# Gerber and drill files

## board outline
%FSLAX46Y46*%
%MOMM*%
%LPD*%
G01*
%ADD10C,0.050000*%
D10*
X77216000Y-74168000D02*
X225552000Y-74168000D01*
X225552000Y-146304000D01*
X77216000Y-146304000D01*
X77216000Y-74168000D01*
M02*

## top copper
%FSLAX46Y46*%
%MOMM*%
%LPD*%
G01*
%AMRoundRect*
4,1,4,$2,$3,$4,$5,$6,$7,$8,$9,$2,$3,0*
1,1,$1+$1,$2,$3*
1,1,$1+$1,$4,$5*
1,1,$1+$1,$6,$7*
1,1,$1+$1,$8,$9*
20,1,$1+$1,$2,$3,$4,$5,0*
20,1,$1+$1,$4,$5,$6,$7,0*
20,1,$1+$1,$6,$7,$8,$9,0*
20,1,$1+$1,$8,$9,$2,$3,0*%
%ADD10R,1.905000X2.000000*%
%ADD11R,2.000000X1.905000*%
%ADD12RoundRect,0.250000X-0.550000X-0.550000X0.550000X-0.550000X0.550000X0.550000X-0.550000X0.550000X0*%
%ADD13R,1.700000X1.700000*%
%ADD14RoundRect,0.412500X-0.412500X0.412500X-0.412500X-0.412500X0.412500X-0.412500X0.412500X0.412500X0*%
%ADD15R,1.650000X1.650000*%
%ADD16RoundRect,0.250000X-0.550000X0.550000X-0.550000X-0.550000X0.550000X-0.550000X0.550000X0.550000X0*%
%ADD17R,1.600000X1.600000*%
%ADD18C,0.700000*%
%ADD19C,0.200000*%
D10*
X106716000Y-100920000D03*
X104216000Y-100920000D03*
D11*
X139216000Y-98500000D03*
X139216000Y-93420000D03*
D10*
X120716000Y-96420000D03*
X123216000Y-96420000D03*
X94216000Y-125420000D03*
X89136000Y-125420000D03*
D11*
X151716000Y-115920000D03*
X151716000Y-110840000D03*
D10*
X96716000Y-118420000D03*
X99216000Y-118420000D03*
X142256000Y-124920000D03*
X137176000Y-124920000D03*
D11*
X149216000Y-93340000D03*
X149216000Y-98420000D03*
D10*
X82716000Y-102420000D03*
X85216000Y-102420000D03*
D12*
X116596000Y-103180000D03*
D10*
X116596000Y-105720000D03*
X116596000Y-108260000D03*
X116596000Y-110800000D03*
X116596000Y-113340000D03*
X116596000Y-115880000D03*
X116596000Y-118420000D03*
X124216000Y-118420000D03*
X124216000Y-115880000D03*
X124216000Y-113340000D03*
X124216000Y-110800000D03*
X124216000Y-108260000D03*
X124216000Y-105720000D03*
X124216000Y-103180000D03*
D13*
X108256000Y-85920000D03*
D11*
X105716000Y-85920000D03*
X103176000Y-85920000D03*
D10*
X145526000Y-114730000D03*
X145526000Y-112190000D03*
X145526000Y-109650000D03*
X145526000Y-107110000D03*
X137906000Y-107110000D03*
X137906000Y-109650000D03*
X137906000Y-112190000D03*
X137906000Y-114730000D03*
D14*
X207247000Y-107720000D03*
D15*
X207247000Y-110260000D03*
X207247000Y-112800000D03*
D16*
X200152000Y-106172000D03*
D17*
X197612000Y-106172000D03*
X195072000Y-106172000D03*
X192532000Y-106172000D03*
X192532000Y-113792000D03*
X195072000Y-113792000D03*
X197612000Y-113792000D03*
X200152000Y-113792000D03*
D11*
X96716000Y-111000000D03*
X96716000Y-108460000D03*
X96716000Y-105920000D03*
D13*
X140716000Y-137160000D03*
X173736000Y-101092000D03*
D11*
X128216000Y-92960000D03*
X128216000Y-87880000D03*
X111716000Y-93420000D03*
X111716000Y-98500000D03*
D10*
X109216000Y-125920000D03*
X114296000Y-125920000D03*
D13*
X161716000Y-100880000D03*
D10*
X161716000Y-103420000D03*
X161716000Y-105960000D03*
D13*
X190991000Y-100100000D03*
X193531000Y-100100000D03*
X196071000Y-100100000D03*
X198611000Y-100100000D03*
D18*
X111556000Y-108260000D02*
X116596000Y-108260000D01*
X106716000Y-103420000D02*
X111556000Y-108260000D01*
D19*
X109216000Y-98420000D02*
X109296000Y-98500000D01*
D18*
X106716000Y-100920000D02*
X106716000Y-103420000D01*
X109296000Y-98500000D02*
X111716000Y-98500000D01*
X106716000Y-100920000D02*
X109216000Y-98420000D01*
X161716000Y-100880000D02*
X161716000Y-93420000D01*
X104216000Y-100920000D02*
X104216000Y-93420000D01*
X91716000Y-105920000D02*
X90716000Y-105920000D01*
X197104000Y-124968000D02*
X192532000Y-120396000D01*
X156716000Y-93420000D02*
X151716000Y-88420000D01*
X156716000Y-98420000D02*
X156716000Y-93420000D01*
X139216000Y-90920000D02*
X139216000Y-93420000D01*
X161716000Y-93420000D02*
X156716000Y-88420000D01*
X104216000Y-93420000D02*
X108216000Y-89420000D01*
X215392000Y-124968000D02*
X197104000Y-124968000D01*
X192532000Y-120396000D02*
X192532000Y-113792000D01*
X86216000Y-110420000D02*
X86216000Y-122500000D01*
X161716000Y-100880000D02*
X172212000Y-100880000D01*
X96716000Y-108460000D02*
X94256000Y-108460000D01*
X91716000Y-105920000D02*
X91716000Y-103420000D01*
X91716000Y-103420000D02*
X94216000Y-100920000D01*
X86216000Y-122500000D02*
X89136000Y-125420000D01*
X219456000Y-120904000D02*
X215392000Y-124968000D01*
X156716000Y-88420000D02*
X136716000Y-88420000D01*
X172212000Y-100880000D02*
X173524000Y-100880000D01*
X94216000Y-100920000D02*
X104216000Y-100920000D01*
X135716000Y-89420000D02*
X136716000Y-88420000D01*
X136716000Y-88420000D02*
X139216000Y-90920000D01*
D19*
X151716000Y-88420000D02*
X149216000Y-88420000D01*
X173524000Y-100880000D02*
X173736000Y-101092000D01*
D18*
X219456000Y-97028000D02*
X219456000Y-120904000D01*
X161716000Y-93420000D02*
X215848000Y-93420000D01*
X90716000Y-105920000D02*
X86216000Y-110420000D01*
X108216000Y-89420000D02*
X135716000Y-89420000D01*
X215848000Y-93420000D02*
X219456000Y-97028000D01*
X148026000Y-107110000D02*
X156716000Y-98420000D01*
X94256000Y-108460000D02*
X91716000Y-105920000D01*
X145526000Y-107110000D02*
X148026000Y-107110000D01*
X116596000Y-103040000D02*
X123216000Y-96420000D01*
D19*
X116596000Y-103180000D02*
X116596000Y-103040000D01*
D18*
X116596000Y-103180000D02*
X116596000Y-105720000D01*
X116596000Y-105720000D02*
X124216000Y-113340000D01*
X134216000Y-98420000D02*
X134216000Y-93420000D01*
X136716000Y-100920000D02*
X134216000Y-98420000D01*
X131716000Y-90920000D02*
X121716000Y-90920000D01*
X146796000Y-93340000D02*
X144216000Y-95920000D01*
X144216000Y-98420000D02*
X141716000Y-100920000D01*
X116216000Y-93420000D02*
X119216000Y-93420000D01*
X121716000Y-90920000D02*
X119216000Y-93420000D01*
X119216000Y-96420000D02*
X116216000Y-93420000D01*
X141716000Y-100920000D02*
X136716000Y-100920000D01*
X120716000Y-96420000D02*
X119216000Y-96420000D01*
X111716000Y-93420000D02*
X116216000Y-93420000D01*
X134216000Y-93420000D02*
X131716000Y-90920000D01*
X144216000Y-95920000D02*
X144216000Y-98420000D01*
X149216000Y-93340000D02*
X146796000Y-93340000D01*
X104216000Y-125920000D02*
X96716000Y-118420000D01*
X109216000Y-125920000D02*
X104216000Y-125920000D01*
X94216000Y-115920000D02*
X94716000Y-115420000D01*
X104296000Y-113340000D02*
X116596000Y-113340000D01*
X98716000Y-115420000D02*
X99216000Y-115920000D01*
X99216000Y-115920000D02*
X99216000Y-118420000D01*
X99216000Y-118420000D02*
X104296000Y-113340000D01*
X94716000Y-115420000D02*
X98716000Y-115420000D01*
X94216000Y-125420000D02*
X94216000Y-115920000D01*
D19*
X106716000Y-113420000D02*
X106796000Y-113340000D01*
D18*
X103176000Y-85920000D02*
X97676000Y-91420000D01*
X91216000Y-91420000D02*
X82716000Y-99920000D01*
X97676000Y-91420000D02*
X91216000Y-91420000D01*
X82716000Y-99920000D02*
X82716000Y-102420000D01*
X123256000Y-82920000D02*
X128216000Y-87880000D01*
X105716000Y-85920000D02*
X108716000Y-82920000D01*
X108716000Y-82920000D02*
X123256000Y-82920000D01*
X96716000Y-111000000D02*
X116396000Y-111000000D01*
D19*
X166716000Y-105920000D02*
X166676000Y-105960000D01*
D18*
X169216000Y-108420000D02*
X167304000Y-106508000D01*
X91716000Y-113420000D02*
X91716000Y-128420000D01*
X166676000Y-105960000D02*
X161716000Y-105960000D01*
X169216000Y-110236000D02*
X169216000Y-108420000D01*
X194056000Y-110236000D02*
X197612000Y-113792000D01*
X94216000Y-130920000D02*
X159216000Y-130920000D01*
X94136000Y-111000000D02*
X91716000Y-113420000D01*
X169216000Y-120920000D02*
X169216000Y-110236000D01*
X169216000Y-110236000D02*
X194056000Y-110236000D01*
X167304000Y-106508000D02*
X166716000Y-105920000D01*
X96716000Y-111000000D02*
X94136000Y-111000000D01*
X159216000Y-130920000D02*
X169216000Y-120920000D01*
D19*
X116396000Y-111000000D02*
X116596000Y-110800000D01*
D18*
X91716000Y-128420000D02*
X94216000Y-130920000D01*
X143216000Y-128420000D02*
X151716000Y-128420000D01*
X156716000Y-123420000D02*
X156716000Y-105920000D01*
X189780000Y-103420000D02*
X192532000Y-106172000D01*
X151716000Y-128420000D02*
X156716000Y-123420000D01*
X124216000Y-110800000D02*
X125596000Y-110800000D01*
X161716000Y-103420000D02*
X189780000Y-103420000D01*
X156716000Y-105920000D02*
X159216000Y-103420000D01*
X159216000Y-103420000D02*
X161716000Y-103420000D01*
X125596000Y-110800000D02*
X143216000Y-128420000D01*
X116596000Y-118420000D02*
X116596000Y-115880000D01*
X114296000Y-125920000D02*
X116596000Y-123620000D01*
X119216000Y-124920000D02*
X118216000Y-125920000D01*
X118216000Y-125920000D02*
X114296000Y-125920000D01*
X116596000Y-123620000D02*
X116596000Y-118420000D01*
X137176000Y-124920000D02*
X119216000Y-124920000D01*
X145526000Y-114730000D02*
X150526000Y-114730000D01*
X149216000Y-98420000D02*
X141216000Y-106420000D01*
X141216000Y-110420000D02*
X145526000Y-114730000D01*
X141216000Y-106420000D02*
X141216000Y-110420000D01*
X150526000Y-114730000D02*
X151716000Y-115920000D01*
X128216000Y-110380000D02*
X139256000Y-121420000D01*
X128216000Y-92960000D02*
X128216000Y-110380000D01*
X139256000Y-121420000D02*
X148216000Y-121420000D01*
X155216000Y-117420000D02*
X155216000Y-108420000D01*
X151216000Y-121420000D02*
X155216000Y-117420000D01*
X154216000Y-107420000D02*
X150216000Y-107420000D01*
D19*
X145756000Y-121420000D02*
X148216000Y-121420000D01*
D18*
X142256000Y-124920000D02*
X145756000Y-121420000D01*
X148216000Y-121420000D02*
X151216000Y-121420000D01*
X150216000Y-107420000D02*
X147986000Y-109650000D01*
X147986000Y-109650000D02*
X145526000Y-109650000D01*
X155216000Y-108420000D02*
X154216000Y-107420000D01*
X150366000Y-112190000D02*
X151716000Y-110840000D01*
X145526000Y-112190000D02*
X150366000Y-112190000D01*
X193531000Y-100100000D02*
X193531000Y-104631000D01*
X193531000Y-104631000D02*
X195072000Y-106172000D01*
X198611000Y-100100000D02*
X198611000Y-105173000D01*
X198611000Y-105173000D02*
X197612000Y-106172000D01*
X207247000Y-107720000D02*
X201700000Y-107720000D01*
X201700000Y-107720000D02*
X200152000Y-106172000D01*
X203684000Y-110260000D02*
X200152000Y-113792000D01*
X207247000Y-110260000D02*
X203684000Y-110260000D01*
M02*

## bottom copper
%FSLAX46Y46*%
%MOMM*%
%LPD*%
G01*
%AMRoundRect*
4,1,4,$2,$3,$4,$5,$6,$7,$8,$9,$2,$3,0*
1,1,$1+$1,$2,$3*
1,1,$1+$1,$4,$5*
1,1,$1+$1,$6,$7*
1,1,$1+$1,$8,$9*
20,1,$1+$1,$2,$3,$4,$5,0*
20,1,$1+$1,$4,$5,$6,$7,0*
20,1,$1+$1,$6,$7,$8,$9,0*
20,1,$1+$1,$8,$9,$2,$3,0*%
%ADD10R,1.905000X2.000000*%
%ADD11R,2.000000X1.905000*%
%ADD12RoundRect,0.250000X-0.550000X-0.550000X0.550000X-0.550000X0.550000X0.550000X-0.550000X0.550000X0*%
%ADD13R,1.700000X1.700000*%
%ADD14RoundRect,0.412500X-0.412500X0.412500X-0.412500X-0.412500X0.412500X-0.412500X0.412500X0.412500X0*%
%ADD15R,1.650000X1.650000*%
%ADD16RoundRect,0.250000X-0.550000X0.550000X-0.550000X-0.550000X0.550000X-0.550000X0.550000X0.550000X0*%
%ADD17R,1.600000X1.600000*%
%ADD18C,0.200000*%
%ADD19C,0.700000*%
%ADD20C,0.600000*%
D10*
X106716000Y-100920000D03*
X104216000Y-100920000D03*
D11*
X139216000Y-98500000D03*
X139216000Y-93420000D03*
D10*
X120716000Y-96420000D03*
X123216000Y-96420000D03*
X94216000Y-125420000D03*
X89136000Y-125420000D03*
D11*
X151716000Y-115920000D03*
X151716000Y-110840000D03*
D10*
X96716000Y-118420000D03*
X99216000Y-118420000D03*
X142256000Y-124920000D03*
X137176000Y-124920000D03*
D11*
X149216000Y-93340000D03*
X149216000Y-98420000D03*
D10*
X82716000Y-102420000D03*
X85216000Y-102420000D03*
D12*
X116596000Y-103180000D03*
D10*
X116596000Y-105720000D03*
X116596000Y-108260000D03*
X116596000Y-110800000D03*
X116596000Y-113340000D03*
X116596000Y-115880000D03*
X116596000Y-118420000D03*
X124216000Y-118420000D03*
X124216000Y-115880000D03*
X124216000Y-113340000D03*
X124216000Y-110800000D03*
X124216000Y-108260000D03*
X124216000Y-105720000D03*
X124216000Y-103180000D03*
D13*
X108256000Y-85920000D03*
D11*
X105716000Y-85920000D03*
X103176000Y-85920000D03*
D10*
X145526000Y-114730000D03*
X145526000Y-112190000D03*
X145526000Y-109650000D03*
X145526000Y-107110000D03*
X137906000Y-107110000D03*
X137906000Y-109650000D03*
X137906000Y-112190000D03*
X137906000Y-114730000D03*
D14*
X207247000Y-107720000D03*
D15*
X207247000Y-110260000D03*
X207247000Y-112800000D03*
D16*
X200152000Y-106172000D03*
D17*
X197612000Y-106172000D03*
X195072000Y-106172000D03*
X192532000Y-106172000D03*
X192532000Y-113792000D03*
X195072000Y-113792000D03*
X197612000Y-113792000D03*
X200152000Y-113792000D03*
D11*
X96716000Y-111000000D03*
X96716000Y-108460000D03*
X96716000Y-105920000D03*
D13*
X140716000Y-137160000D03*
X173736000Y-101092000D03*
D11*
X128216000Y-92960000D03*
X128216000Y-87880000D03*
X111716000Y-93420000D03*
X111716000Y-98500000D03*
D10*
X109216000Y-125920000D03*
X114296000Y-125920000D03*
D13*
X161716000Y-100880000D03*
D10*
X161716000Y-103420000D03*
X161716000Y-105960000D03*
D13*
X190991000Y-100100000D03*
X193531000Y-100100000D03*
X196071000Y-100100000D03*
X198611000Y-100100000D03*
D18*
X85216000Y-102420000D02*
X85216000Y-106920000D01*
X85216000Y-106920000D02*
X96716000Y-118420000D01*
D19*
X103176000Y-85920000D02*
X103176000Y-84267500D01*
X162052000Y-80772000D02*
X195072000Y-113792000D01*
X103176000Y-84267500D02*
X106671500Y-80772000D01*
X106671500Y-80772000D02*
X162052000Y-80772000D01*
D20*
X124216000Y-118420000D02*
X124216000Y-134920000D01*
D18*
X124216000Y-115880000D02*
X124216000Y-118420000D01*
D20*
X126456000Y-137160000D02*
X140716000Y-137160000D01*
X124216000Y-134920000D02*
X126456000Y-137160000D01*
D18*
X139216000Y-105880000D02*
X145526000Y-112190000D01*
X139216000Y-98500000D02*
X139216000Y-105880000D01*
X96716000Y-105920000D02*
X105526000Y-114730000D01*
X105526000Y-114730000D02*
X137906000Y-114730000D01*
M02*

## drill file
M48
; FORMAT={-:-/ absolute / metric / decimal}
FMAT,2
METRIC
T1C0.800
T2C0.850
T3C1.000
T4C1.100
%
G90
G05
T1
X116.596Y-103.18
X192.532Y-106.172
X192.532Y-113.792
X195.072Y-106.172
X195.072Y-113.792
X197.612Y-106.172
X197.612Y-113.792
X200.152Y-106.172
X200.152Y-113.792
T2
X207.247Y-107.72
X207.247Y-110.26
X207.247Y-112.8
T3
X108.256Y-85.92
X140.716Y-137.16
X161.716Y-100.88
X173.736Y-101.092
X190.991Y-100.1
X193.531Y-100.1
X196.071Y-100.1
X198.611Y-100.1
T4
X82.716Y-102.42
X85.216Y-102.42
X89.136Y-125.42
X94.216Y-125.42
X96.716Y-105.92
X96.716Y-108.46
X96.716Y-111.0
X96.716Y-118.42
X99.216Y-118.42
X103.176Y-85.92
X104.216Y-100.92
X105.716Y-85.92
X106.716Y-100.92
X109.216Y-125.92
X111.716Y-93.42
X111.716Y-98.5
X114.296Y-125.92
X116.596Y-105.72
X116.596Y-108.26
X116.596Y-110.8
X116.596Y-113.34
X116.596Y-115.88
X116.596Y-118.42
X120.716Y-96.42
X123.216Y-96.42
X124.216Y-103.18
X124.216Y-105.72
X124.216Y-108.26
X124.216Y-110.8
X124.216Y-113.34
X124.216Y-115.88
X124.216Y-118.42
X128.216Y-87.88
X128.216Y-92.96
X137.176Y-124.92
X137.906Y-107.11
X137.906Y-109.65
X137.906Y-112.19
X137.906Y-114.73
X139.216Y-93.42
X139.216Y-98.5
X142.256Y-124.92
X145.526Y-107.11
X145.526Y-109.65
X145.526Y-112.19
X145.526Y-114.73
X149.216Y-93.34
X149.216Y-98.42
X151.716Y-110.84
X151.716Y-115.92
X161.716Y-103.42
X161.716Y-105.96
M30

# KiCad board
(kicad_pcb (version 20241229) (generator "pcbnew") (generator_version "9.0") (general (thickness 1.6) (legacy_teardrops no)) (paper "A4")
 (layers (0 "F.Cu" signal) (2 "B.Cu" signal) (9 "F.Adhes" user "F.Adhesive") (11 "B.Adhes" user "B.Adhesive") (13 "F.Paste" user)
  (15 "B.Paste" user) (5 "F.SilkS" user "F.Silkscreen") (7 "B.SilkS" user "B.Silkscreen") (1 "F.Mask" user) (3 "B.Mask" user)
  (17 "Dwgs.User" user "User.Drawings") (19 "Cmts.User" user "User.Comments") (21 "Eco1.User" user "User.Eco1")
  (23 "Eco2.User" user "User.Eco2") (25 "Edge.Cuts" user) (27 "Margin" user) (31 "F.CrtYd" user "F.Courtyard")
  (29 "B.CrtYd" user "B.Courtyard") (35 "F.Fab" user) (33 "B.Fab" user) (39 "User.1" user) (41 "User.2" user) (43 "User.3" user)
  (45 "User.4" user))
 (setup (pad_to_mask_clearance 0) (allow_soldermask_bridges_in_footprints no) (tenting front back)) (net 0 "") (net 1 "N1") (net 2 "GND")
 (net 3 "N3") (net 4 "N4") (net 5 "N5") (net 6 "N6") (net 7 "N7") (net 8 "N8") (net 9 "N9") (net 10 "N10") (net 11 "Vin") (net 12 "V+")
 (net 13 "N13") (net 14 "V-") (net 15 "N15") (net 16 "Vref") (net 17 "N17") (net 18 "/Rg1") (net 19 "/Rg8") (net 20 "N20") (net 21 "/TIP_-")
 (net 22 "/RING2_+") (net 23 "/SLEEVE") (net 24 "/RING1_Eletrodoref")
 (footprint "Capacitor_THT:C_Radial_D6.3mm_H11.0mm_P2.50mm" (layer "F.Cu") (at 106.716 100.92 180)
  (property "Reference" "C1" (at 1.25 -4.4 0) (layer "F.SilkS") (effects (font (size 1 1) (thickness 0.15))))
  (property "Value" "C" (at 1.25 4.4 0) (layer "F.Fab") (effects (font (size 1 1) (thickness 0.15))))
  (pad "1" thru_hole rect (at 0 0 180) (size 1.905 2) (drill 1.1) (layers "*.Cu" "*.Mask") (remove_unused_layers no) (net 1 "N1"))
  (pad "2" thru_hole rect (at 2.5 0 180) (size 1.905 2) (drill 1.1) (layers "*.Cu" "*.Mask") (remove_unused_layers no) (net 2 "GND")))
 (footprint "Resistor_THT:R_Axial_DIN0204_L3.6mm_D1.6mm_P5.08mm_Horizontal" (layer "F.Cu") (at 139.216 98.5 90)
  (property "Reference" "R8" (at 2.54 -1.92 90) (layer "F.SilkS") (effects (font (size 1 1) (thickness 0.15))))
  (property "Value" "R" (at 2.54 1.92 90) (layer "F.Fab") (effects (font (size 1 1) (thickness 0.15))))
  (pad "1" thru_hole rect (at 0 0 90) (size 1.905 2) (drill 1.1) (layers "*.Cu" "*.Mask") (remove_unused_layers no) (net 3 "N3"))
  (pad "2" thru_hole rect (at 5.08 0 90) (size 1.905 2) (drill 1.1) (layers "*.Cu" "*.Mask") (remove_unused_layers no) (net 2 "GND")))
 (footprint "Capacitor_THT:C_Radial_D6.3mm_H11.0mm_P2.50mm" (layer "F.Cu") (at 120.716 96.42)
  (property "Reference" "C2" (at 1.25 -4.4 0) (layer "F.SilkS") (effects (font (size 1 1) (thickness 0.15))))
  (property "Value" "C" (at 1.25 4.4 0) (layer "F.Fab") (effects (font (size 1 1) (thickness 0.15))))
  (pad "1" thru_hole rect (at 0 0) (size 1.905 2) (drill 1.1) (layers "*.Cu" "*.Mask") (remove_unused_layers no) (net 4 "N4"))
  (pad "2" thru_hole rect (at 2.5 0) (size 1.905 2) (drill 1.1) (layers "*.Cu" "*.Mask") (remove_unused_layers no) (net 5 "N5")))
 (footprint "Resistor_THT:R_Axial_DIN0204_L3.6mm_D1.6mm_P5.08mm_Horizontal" (layer "F.Cu") (at 94.216 125.42 180)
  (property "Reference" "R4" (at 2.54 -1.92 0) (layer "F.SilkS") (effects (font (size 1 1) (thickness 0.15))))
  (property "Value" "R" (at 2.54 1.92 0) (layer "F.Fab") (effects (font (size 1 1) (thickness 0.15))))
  (pad "1" thru_hole rect (at 0 0 180) (size 1.905 2) (drill 1.1) (layers "*.Cu" "*.Mask") (remove_unused_layers no) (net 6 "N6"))
  (pad "2" thru_hole rect (at 5.08 0 180) (size 1.905 2) (drill 1.1) (layers "*.Cu" "*.Mask") (remove_unused_layers no) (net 2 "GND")))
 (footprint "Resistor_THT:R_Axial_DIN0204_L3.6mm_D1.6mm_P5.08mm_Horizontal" (layer "F.Cu") (at 151.716 115.92 90)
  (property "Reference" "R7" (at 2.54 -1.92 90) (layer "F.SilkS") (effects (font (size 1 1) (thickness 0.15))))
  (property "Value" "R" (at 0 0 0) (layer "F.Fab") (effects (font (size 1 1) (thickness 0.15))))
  (pad "1" thru_hole rect (at 0 0 90) (size 1.905 2) (drill 1.1) (layers "*.Cu" "*.Mask") (remove_unused_layers no) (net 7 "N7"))
  (pad "2" thru_hole rect (at 5.08 0 90) (size 1.905 2) (drill 1.1) (layers "*.Cu" "*.Mask") (remove_unused_layers no) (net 3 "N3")))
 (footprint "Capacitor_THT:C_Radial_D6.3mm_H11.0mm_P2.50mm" (layer "F.Cu") (at 96.716 118.42)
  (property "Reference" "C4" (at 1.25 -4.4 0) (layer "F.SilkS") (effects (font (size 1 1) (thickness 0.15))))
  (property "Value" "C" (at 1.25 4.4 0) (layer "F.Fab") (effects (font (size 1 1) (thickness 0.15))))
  (pad "1" thru_hole rect (at 0 0) (size 1.905 2) (drill 1.1) (layers "*.Cu" "*.Mask") (remove_unused_layers no) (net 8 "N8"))
  (pad "2" thru_hole rect (at 2.5 0) (size 1.905 2) (drill 1.1) (layers "*.Cu" "*.Mask") (remove_unused_layers no) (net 6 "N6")))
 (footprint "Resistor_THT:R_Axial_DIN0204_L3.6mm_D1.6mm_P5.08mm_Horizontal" (layer "F.Cu") (at 142.256 124.92 180)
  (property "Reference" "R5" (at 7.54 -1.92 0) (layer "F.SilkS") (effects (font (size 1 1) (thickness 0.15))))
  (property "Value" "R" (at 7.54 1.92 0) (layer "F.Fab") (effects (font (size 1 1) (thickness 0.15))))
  (pad "1" thru_hole rect (at 0 0 180) (size 1.905 2) (drill 1.1) (layers "*.Cu" "*.Mask") (remove_unused_layers no) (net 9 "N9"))
  (pad "2" thru_hole rect (at 5.08 0 180) (size 1.905 2) (drill 1.1) (layers "*.Cu" "*.Mask") (remove_unused_layers no) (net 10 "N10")))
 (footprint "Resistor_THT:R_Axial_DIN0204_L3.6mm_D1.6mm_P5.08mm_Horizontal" (layer "F.Cu") (at 149.216 93.34 -90)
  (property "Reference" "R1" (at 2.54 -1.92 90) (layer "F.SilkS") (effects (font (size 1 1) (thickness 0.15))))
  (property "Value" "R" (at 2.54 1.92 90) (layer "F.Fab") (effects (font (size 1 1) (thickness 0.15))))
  (pad "1" thru_hole rect (at 0 0 270) (size 1.905 2) (drill 1.1) (layers "*.Cu" "*.Mask") (remove_unused_layers no) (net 4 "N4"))
  (pad "2" thru_hole rect (at 5.08 0 270) (size 1.905 2) (drill 1.1) (layers "*.Cu" "*.Mask") (remove_unused_layers no) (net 7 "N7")))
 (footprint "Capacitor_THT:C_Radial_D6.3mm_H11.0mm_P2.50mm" (layer "F.Cu") (at 82.716 102.42)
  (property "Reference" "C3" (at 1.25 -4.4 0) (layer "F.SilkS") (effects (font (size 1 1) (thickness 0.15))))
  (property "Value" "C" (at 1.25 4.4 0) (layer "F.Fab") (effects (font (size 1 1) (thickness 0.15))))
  (pad "1" thru_hole rect (at 0 0) (size 1.905 2) (drill 1.1) (layers "*.Cu" "*.Mask") (remove_unused_layers no) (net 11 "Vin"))
  (pad "2" thru_hole rect (at 2.5 0) (size 1.905 2) (drill 1.1) (layers "*.Cu" "*.Mask") (remove_unused_layers no) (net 8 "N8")))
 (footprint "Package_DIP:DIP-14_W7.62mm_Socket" (layer "F.Cu") (at 116.596 103.18)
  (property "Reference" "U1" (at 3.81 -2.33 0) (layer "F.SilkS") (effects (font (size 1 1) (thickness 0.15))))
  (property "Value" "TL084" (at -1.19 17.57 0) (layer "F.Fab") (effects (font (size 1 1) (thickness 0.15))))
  (pad "1" thru_hole roundrect (at 0 0) (size 1.6 1.6) (drill 0.8) (layers "*.Cu" "*.Mask") (remove_unused_layers no)
   (roundrect_rratio 0.15625) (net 5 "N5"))
  (pad "2" thru_hole rect (at 0 2.54) (size 1.905 2) (drill 1.1) (layers "*.Cu" "*.Mask") (remove_unused_layers no) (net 5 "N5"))
  (pad "3" thru_hole rect (at 0 5.08) (size 1.905 2) (drill 1.1) (layers "*.Cu" "*.Mask") (remove_unused_layers no) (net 1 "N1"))
  (pad "4" thru_hole rect (at 0 7.62) (size 1.905 2) (drill 1.1) (layers "*.Cu" "*.Mask") (remove_unused_layers no) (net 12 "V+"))
  (pad "5" thru_hole rect (at 0 10.16) (size 1.905 2) (drill 1.1) (layers "*.Cu" "*.Mask") (remove_unused_layers no) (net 6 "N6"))
  (pad "6" thru_hole rect (at 0 12.7) (size 1.905 2) (drill 1.1) (layers "*.Cu" "*.Mask") (remove_unused_layers no) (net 10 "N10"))
  (pad "7" thru_hole rect (at 0 15.24) (size 1.905 2) (drill 1.1) (layers "*.Cu" "*.Mask") (remove_unused_layers no) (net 10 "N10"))
  (pad "8" thru_hole rect (at 7.62 15.24) (size 1.905 2) (drill 1.1) (layers "*.Cu" "*.Mask") (remove_unused_layers no) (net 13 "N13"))
  (pad "9" thru_hole rect (at 7.62 12.7) (size 1.905 2) (drill 1.1) (layers "*.Cu" "*.Mask") (remove_unused_layers no) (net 13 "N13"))
  (pad "10" thru_hole rect (at 7.62 10.16) (size 1.905 2) (drill 1.1) (layers "*.Cu" "*.Mask") (remove_unused_layers no) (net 5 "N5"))
  (pad "11" thru_hole rect (at 7.62 7.62) (size 1.905 2) (drill 1.1) (layers "*.Cu" "*.Mask") (remove_unused_layers no) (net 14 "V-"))
  (pad "12" thru_hole rect (at 7.62 5.08) (size 1.905 2) (drill 1.1) (layers "*.Cu" "*.Mask") (remove_unused_layers no))
  (pad "13" thru_hole rect (at 7.62 2.54) (size 1.905 2) (drill 1.1) (layers "*.Cu" "*.Mask") (remove_unused_layers no))
  (pad "14" thru_hole rect (at 7.62 0) (size 1.905 2) (drill 1.1) (layers "*.Cu" "*.Mask") (remove_unused_layers no)))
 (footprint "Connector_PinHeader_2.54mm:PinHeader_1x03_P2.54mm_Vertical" (layer "F.Cu") (at 108.256 85.92 -90)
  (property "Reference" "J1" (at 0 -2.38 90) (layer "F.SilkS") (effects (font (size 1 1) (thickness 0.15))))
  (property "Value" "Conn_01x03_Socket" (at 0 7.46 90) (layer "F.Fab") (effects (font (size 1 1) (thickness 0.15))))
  (pad "1" thru_hole rect (at 0 0 270) (size 1.7 1.7) (drill 1) (layers "*.Cu" "*.Mask") (remove_unused_layers no) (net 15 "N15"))
  (pad "2" thru_hole rect (at 0 2.54 270) (size 1.905 2) (drill 1.1) (layers "*.Cu" "*.Mask") (remove_unused_layers no) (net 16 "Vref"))
  (pad "3" thru_hole rect (at 0 5.08 270) (size 1.905 2) (drill 1.1) (layers "*.Cu" "*.Mask") (remove_unused_layers no) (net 11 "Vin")))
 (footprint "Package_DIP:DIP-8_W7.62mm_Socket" (layer "F.Cu") (at 145.526 114.73 180)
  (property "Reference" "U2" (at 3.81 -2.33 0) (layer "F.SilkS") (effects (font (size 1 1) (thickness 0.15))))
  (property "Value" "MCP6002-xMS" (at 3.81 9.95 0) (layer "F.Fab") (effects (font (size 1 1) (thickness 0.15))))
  (pad "1" thru_hole rect (at 0 0 180) (size 1.905 2) (drill 1.1) (layers "*.Cu" "*.Mask") (remove_unused_layers no) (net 7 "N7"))
  (pad "2" thru_hole rect (at 0 2.54 180) (size 1.905 2) (drill 1.1) (layers "*.Cu" "*.Mask") (remove_unused_layers no) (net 3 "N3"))
  (pad "3" thru_hole rect (at 0 5.08 180) (size 1.905 2) (drill 1.1) (layers "*.Cu" "*.Mask") (remove_unused_layers no) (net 9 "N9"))
  (pad "4" thru_hole rect (at 0 7.62 180) (size 1.905 2) (drill 1.1) (layers "*.Cu" "*.Mask") (remove_unused_layers no) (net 2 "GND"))
  (pad "5" thru_hole rect (at 7.62 7.62 180) (size 1.905 2) (drill 1.1) (layers "*.Cu" "*.Mask") (remove_unused_layers no))
  (pad "6" thru_hole rect (at 7.62 5.08 180) (size 1.905 2) (drill 1.1) (layers "*.Cu" "*.Mask") (remove_unused_layers no))
  (pad "7" thru_hole rect (at 7.62 2.54 180) (size 1.905 2) (drill 1.1) (layers "*.Cu" "*.Mask") (remove_unused_layers no))
  (pad "8" thru_hole rect (at 7.62 0 180) (size 1.905 2) (drill 1.1) (layers "*.Cu" "*.Mask") (remove_unused_layers no) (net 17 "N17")))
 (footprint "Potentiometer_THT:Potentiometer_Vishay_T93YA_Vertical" (layer "F.Cu") (at 207.247 107.72 -90)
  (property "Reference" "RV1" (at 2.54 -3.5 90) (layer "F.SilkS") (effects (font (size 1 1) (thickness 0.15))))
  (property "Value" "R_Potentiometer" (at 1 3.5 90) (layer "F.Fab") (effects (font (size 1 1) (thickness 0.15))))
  (pad "1" thru_hole roundrect (at 0 0 270) (size 1.65 1.65) (drill 0.85) (layers "*.Cu" "*.Mask") (remove_unused_layers no)
   (roundrect_rratio 0.25) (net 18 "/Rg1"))
  (pad "2" thru_hole rect (at 2.54 0 270) (size 1.65 1.65) (drill 0.85) (layers "*.Cu" "*.Mask") (remove_unused_layers no) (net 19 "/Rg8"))
  (pad "3" thru_hole rect (at 5.08 0 270) (size 1.65 1.65) (drill 0.85) (layers "*.Cu" "*.Mask") (remove_unused_layers no) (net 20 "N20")))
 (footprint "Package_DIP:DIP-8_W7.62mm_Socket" (layer "F.Cu") (at 200.152 106.172 -90)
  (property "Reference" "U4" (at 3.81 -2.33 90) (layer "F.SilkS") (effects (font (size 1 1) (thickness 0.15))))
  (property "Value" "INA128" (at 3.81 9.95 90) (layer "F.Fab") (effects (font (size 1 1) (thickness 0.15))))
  (pad "1" thru_hole roundrect (at 0 0 270) (size 1.6 1.6) (drill 0.8) (layers "*.Cu" "*.Mask") (remove_unused_layers no)
   (roundrect_rratio 0.15625) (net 18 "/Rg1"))
  (pad "2" thru_hole rect (at 0 2.54 270) (size 1.6 1.6) (drill 0.8) (layers "*.Cu" "*.Mask") (remove_unused_layers no) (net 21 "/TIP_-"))
  (pad "3" thru_hole rect (at 0 5.08 270) (size 1.6 1.6) (drill 0.8) (layers "*.Cu" "*.Mask") (remove_unused_layers no) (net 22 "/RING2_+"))
  (pad "4" thru_hole rect (at 0 7.62 270) (size 1.6 1.6) (drill 0.8) (layers "*.Cu" "*.Mask") (remove_unused_layers no) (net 14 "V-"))
  (pad "5" thru_hole rect (at 7.62 7.62 270) (size 1.6 1.6) (drill 0.8) (layers "*.Cu" "*.Mask") (remove_unused_layers no) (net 2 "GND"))
  (pad "6" thru_hole rect (at 7.62 5.08 270) (size 1.6 1.6) (drill 0.8) (layers "*.Cu" "*.Mask") (remove_unused_layers no) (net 11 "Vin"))
  (pad "7" thru_hole rect (at 7.62 2.54 270) (size 1.6 1.6) (drill 0.8) (layers "*.Cu" "*.Mask") (remove_unused_layers no) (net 12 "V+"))
  (pad "8" thru_hole rect (at 7.62 0 270) (size 1.6 1.6) (drill 0.8) (layers "*.Cu" "*.Mask") (remove_unused_layers no) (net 19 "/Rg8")))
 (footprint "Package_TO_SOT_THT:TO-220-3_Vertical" (layer "F.Cu") (at 96.716 111 90)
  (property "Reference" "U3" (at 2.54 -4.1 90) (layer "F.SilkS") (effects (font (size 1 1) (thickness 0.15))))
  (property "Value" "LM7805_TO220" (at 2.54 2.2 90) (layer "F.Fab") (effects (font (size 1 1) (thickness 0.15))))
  (pad "1" thru_hole rect (at 0 0 90) (size 1.905 2) (drill 1.1) (layers "*.Cu" "*.Mask") (remove_unused_layers no) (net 12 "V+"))
  (pad "2" thru_hole rect (at 2.54 0 90) (size 1.905 2) (drill 1.1) (layers "*.Cu" "*.Mask") (remove_unused_layers no) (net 2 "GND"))
  (pad "3" thru_hole rect (at 5.08 0 90) (size 1.905 2) (drill 1.1) (layers "*.Cu" "*.Mask") (remove_unused_layers no) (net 17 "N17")))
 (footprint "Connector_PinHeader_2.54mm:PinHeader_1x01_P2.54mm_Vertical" (layer "F.Cu") (at 140.716 137.16)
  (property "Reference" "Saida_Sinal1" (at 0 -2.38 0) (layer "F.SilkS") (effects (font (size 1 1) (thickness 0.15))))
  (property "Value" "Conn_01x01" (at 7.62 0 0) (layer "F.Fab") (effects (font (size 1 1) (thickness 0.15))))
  (pad "1" thru_hole rect (at 0 0) (size 1.7 1.7) (drill 1) (layers "*.Cu" "*.Mask") (remove_unused_layers no) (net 13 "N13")))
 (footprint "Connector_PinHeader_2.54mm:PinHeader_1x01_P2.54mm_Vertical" (layer "F.Cu") (at 173.736 101.092)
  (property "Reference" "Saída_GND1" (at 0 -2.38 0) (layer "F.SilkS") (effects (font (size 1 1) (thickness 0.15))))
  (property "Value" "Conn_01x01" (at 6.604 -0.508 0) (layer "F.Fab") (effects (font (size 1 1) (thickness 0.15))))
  (pad "1" thru_hole rect (at 0 0) (size 1.7 1.7) (drill 1) (layers "*.Cu" "*.Mask") (remove_unused_layers no) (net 2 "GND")))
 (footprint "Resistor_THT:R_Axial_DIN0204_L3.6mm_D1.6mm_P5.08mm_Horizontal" (layer "F.Cu") (at 128.216 92.96 90)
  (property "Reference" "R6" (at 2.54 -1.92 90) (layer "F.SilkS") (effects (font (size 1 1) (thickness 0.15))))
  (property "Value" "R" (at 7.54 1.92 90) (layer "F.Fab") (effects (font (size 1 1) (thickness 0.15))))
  (pad "1" thru_hole rect (at 0 0 90) (size 1.905 2) (drill 1.1) (layers "*.Cu" "*.Mask") (remove_unused_layers no) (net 9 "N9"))
  (pad "2" thru_hole rect (at 5.08 0 90) (size 1.905 2) (drill 1.1) (layers "*.Cu" "*.Mask") (remove_unused_layers no) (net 16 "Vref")))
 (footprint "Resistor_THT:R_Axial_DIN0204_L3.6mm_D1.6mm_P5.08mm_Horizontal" (layer "F.Cu") (at 111.716 93.42 -90)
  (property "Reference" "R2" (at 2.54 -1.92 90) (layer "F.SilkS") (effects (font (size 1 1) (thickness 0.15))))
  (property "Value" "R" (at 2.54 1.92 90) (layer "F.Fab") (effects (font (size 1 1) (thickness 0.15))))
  (pad "1" thru_hole rect (at 0 0 270) (size 1.905 2) (drill 1.1) (layers "*.Cu" "*.Mask") (remove_unused_layers no) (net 4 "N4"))
  (pad "2" thru_hole rect (at 5.08 0 270) (size 1.905 2) (drill 1.1) (layers "*.Cu" "*.Mask") (remove_unused_layers no) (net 1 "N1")))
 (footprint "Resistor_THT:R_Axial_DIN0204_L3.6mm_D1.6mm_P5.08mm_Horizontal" (layer "F.Cu") (at 109.216 125.92)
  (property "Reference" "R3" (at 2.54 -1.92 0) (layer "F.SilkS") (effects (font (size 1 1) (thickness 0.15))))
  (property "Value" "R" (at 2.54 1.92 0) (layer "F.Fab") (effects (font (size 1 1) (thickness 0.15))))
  (pad "1" thru_hole rect (at 0 0) (size 1.905 2) (drill 1.1) (layers "*.Cu" "*.Mask") (remove_unused_layers no) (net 8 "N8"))
  (pad "2" thru_hole rect (at 5.08 0) (size 1.905 2) (drill 1.1) (layers "*.Cu" "*.Mask") (remove_unused_layers no) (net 10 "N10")))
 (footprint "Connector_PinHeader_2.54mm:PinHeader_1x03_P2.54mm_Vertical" (layer "F.Cu") (at 161.716 100.88)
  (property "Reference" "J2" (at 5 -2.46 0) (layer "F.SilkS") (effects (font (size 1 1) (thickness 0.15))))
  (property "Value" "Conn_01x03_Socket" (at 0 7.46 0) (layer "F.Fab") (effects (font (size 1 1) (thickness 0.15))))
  (pad "1" thru_hole rect (at 0 0) (size 1.7 1.7) (drill 1) (layers "*.Cu" "*.Mask") (remove_unused_layers no) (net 2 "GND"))
  (pad "2" thru_hole rect (at 0 2.54) (size 1.905 2) (drill 1.1) (layers "*.Cu" "*.Mask") (remove_unused_layers no) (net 14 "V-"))
  (pad "3" thru_hole rect (at 0 5.08) (size 1.905 2) (drill 1.1) (layers "*.Cu" "*.Mask") (remove_unused_layers no) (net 12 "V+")))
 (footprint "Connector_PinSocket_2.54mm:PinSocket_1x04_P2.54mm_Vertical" (layer "F.Cu") (at 190.991 100.1 90)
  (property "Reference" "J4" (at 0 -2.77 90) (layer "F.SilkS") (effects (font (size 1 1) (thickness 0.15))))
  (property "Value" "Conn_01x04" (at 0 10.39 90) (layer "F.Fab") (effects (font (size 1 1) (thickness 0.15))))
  (pad "1" thru_hole rect (at 0 0 90) (size 1.7 1.7) (drill 1) (layers "*.Cu" "*.Mask") (remove_unused_layers no) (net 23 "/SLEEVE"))
  (pad "2" thru_hole rect (at 0 2.54 90) (size 1.7 1.7) (drill 1) (layers "*.Cu" "*.Mask") (remove_unused_layers no) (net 22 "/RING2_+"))
  (pad "3" thru_hole rect (at 0 5.08 90) (size 1.7 1.7) (drill 1) (layers "*.Cu" "*.Mask") (remove_unused_layers no)
   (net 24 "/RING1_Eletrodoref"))
  (pad "4" thru_hole rect (at 0 7.62 90) (size 1.7 1.7) (drill 1) (layers "*.Cu" "*.Mask") (remove_unused_layers no) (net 21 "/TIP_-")))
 (gr_rect (start 77.216 74.168) (end 225.552 146.304) (stroke (width 0.05) (type default)) (fill no) (layer "Edge.Cuts"))
 (segment (start 111.556 108.26) (end 116.596 108.26) (width 0.7) (layer "F.Cu") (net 1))
 (segment (start 106.716 103.42) (end 111.556 108.26) (width 0.7) (layer "F.Cu") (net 1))
 (segment (start 109.216 98.42) (end 109.296 98.5) (width 0.2) (layer "F.Cu") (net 1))
 (segment (start 106.716 100.92) (end 106.716 103.42) (width 0.7) (layer "F.Cu") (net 1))
 (segment (start 109.296 98.5) (end 111.716 98.5) (width 0.7) (layer "F.Cu") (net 1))
 (segment (start 106.716 100.92) (end 109.216 98.42) (width 0.7) (layer "F.Cu") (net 1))
 (segment (start 161.716 100.88) (end 161.716 93.42) (width 0.7) (layer "F.Cu") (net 2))
 (segment (start 104.216 100.92) (end 104.216 93.42) (width 0.7) (layer "F.Cu") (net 2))
 (segment (start 91.716 105.92) (end 90.716 105.92) (width 0.7) (layer "F.Cu") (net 2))
 (segment (start 197.104 124.968) (end 192.532 120.396) (width 0.7) (layer "F.Cu") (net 2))
 (segment (start 156.716 93.42) (end 151.716 88.42) (width 0.7) (layer "F.Cu") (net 2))
 (segment (start 156.716 98.42) (end 156.716 93.42) (width 0.7) (layer "F.Cu") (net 2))
 (segment (start 139.216 90.92) (end 139.216 93.42) (width 0.7) (layer "F.Cu") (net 2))
 (segment (start 161.716 93.42) (end 156.716 88.42) (width 0.7) (layer "F.Cu") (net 2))
 (segment (start 104.216 93.42) (end 108.216 89.42) (width 0.7) (layer "F.Cu") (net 2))
 (segment (start 215.392 124.968) (end 197.104 124.968) (width 0.7) (layer "F.Cu") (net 2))
 (segment (start 192.532 120.396) (end 192.532 113.792) (width 0.7) (layer "F.Cu") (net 2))
 (segment (start 86.216 110.42) (end 86.216 122.5) (width 0.7) (layer "F.Cu") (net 2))
 (segment (start 161.716 100.88) (end 172.212 100.88) (width 0.7) (layer "F.Cu") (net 2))
 (segment (start 96.716 108.46) (end 94.256 108.46) (width 0.7) (layer "F.Cu") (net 2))
 (segment (start 91.716 105.92) (end 91.716 103.42) (width 0.7) (layer "F.Cu") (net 2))
 (segment (start 91.716 103.42) (end 94.216 100.92) (width 0.7) (layer "F.Cu") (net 2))
 (segment (start 86.216 122.5) (end 89.136 125.42) (width 0.7) (layer "F.Cu") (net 2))
 (segment (start 219.456 120.904) (end 215.392 124.968) (width 0.7) (layer "F.Cu") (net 2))
 (segment (start 156.716 88.42) (end 136.716 88.42) (width 0.7) (layer "F.Cu") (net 2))
 (segment (start 172.212 100.88) (end 173.524 100.88) (width 0.7) (layer "F.Cu") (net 2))
 (segment (start 94.216 100.92) (end 104.216 100.92) (width 0.7) (layer "F.Cu") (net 2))
 (segment (start 135.716 89.42) (end 136.716 88.42) (width 0.7) (layer "F.Cu") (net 2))
 (segment (start 136.716 88.42) (end 139.216 90.92) (width 0.7) (layer "F.Cu") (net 2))
 (segment (start 151.716 88.42) (end 149.216 88.42) (width 0.2) (layer "F.Cu") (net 2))
 (segment (start 173.524 100.88) (end 173.736 101.092) (width 0.2) (layer "F.Cu") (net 2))
 (segment (start 219.456 97.028) (end 219.456 120.904) (width 0.7) (layer "F.Cu") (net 2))
 (segment (start 161.716 93.42) (end 215.848 93.42) (width 0.7) (layer "F.Cu") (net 2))
 (segment (start 90.716 105.92) (end 86.216 110.42) (width 0.7) (layer "F.Cu") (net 2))
 (segment (start 108.216 89.42) (end 135.716 89.42) (width 0.7) (layer "F.Cu") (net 2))
 (segment (start 215.848 93.42) (end 219.456 97.028) (width 0.7) (layer "F.Cu") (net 2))
 (segment (start 148.026 107.11) (end 156.716 98.42) (width 0.7) (layer "F.Cu") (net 2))
 (segment (start 94.256 108.46) (end 91.716 105.92) (width 0.7) (layer "F.Cu") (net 2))
 (segment (start 145.526 107.11) (end 148.026 107.11) (width 0.7) (layer "F.Cu") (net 2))
 (segment (start 116.596 103.04) (end 123.216 96.42) (width 0.7) (layer "F.Cu") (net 5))
 (segment (start 116.596 103.18) (end 116.596 103.04) (width 0.2) (layer "F.Cu") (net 5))
 (segment (start 116.596 103.18) (end 116.596 105.72) (width 0.7) (layer "F.Cu") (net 5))
 (segment (start 116.596 105.72) (end 124.216 113.34) (width 0.7) (layer "F.Cu") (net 5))
 (segment (start 134.216 98.42) (end 134.216 93.42) (width 0.7) (layer "F.Cu") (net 4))
 (segment (start 136.716 100.92) (end 134.216 98.42) (width 0.7) (layer "F.Cu") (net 4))
 (segment (start 131.716 90.92) (end 121.716 90.92) (width 0.7) (layer "F.Cu") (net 4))
 (segment (start 146.796 93.34) (end 144.216 95.92) (width 0.7) (layer "F.Cu") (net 4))
 (segment (start 144.216 98.42) (end 141.716 100.92) (width 0.7) (layer "F.Cu") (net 4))
 (segment (start 116.216 93.42) (end 119.216 93.42) (width 0.7) (layer "F.Cu") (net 4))
 (segment (start 121.716 90.92) (end 119.216 93.42) (width 0.7) (layer "F.Cu") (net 4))
 (segment (start 119.216 96.42) (end 116.216 93.42) (width 0.7) (layer "F.Cu") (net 4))
 (segment (start 141.716 100.92) (end 136.716 100.92) (width 0.7) (layer "F.Cu") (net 4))
 (segment (start 120.716 96.42) (end 119.216 96.42) (width 0.7) (layer "F.Cu") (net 4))
 (segment (start 111.716 93.42) (end 116.216 93.42) (width 0.7) (layer "F.Cu") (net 4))
 (segment (start 134.216 93.42) (end 131.716 90.92) (width 0.7) (layer "F.Cu") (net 4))
 (segment (start 144.216 95.92) (end 144.216 98.42) (width 0.7) (layer "F.Cu") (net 4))
 (segment (start 149.216 93.34) (end 146.796 93.34) (width 0.7) (layer "F.Cu") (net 4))
 (segment (start 104.216 125.92) (end 96.716 118.42) (width 0.7) (layer "F.Cu") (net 8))
 (segment (start 109.216 125.92) (end 104.216 125.92) (width 0.7) (layer "F.Cu") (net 8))
 (segment (start 85.216 102.42) (end 85.216 106.92) (width 0.2) (layer "B.Cu") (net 8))
 (segment (start 85.216 106.92) (end 96.716 118.42) (width 0.2) (layer "B.Cu") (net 8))
 (segment (start 94.216 115.92) (end 94.716 115.42) (width 0.7) (layer "F.Cu") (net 6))
 (segment (start 104.296 113.34) (end 116.596 113.34) (width 0.7) (layer "F.Cu") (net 6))
 (segment (start 98.716 115.42) (end 99.216 115.92) (width 0.7) (layer "F.Cu") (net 6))
 (segment (start 99.216 115.92) (end 99.216 118.42) (width 0.7) (layer "F.Cu") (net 6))
 (segment (start 99.216 118.42) (end 104.296 113.34) (width 0.7) (layer "F.Cu") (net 6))
 (segment (start 94.716 115.42) (end 98.716 115.42) (width 0.7) (layer "F.Cu") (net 6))
 (segment (start 94.216 125.42) (end 94.216 115.92) (width 0.7) (layer "F.Cu") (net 6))
 (segment (start 106.716 113.42) (end 106.796 113.34) (width 0.2) (layer "F.Cu") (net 6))
 (segment (start 103.176 85.92) (end 97.676 91.42) (width 0.7) (layer "F.Cu") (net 11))
 (segment (start 91.216 91.42) (end 82.716 99.92) (width 0.7) (layer "F.Cu") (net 11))
 (segment (start 97.676 91.42) (end 91.216 91.42) (width 0.7) (layer "F.Cu") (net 11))
 (segment (start 82.716 99.92) (end 82.716 102.42) (width 0.7) (layer "F.Cu") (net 11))
 (segment (start 103.176 85.92) (end 103.176 84.2675) (width 0.7) (layer "B.Cu") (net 11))
 (segment (start 162.052 80.772) (end 195.072 113.792) (width 0.7) (layer "B.Cu") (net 11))
 (segment (start 103.176 84.2675) (end 106.6715 80.772) (width 0.7) (layer "B.Cu") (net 11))
 (segment (start 106.6715 80.772) (end 162.052 80.772) (width 0.7) (layer "B.Cu") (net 11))
 (segment (start 123.256 82.92) (end 128.216 87.88) (width 0.7) (layer "F.Cu") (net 16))
 (segment (start 105.716 85.92) (end 108.716 82.92) (width 0.7) (layer "F.Cu") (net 16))
 (segment (start 108.716 82.92) (end 123.256 82.92) (width 0.7) (layer "F.Cu") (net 16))
 (segment (start 96.716 111) (end 116.396 111) (width 0.7) (layer "F.Cu") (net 12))
 (segment (start 166.716 105.92) (end 166.676 105.96) (width 0.2) (layer "F.Cu") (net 12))
 (segment (start 169.216 108.42) (end 167.304 106.508) (width 0.7) (layer "F.Cu") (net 12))
 (segment (start 91.716 113.42) (end 91.716 128.42) (width 0.7) (layer "F.Cu") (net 12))
 (segment (start 166.676 105.96) (end 161.716 105.96) (width 0.7) (layer "F.Cu") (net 12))
 (segment (start 169.216 110.236) (end 169.216 108.42) (width 0.7) (layer "F.Cu") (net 12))
 (segment (start 194.056 110.236) (end 197.612 113.792) (width 0.7) (layer "F.Cu") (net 12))
 (segment (start 94.216 130.92) (end 159.216 130.92) (width 0.7) (layer "F.Cu") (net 12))
 (segment (start 94.136 111) (end 91.716 113.42) (width 0.7) (layer "F.Cu") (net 12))
 (segment (start 169.216 120.92) (end 169.216 110.236) (width 0.7) (layer "F.Cu") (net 12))
 (segment (start 169.216 110.236) (end 194.056 110.236) (width 0.7) (layer "F.Cu") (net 12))
 (segment (start 167.304 106.508) (end 166.716 105.92) (width 0.7) (layer "F.Cu") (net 12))
 (segment (start 96.716 111) (end 94.136 111) (width 0.7) (layer "F.Cu") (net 12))
 (segment (start 159.216 130.92) (end 169.216 120.92) (width 0.7) (layer "F.Cu") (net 12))
 (segment (start 116.396 111) (end 116.596 110.8) (width 0.2) (layer "F.Cu") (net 12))
 (segment (start 91.716 128.42) (end 94.216 130.92) (width 0.7) (layer "F.Cu") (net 12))
 (segment (start 143.216 128.42) (end 151.716 128.42) (width 0.7) (layer "F.Cu") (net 14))
 (segment (start 156.716 123.42) (end 156.716 105.92) (width 0.7) (layer "F.Cu") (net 14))
 (segment (start 189.78 103.42) (end 192.532 106.172) (width 0.7) (layer "F.Cu") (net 14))
 (segment (start 151.716 128.42) (end 156.716 123.42) (width 0.7) (layer "F.Cu") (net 14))
 (segment (start 124.216 110.8) (end 125.596 110.8) (width 0.7) (layer "F.Cu") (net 14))
 (segment (start 161.716 103.42) (end 189.78 103.42) (width 0.7) (layer "F.Cu") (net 14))
 (segment (start 156.716 105.92) (end 159.216 103.42) (width 0.7) (layer "F.Cu") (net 14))
 (segment (start 159.216 103.42) (end 161.716 103.42) (width 0.7) (layer "F.Cu") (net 14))
 (segment (start 125.596 110.8) (end 143.216 128.42) (width 0.7) (layer "F.Cu") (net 14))
 (segment (start 124.216 118.42) (end 124.216 134.92) (width 0.6) (layer "B.Cu") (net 13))
 (segment (start 124.216 115.88) (end 124.216 118.42) (width 0.2) (layer "B.Cu") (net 13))
 (segment (start 126.456 137.16) (end 140.716 137.16) (width 0.6) (layer "B.Cu") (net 13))
 (segment (start 124.216 134.92) (end 126.456 137.16) (width 0.6) (layer "B.Cu") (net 13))
 (segment (start 116.596 118.42) (end 116.596 115.88) (width 0.7) (layer "F.Cu") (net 10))
 (segment (start 114.296 125.92) (end 116.596 123.62) (width 0.7) (layer "F.Cu") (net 10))
 (segment (start 119.216 124.92) (end 118.216 125.92) (width 0.7) (layer "F.Cu") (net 10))
 (segment (start 118.216 125.92) (end 114.296 125.92) (width 0.7) (layer "F.Cu") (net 10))
 (segment (start 116.596 123.62) (end 116.596 118.42) (width 0.7) (layer "F.Cu") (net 10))
 (segment (start 137.176 124.92) (end 119.216 124.92) (width 0.7) (layer "F.Cu") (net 10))
 (segment (start 145.526 114.73) (end 150.526 114.73) (width 0.7) (layer "F.Cu") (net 7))
 (segment (start 149.216 98.42) (end 141.216 106.42) (width 0.7) (layer "F.Cu") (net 7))
 (segment (start 141.216 110.42) (end 145.526 114.73) (width 0.7) (layer "F.Cu") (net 7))
 (segment (start 141.216 106.42) (end 141.216 110.42) (width 0.7) (layer "F.Cu") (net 7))
 (segment (start 150.526 114.73) (end 151.716 115.92) (width 0.7) (layer "F.Cu") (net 7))
 (segment (start 128.216 110.38) (end 139.256 121.42) (width 0.7) (layer "F.Cu") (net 9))
 (segment (start 128.216 92.96) (end 128.216 110.38) (width 0.7) (layer "F.Cu") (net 9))
 (segment (start 139.256 121.42) (end 148.216 121.42) (width 0.7) (layer "F.Cu") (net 9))
 (segment (start 155.216 117.42) (end 155.216 108.42) (width 0.7) (layer "F.Cu") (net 9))
 (segment (start 151.216 121.42) (end 155.216 117.42) (width 0.7) (layer "F.Cu") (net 9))
 (segment (start 154.216 107.42) (end 150.216 107.42) (width 0.7) (layer "F.Cu") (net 9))
 (segment (start 145.756 121.42) (end 148.216 121.42) (width 0.2) (layer "F.Cu") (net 9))
 (segment (start 142.256 124.92) (end 145.756 121.42) (width 0.7) (layer "F.Cu") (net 9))
 (segment (start 148.216 121.42) (end 151.216 121.42) (width 0.7) (layer "F.Cu") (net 9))
 (segment (start 150.216 107.42) (end 147.986 109.65) (width 0.7) (layer "F.Cu") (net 9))
 (segment (start 147.986 109.65) (end 145.526 109.65) (width 0.7) (layer "F.Cu") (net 9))
 (segment (start 155.216 108.42) (end 154.216 107.42) (width 0.7) (layer "F.Cu") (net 9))
 (segment (start 150.366 112.19) (end 151.716 110.84) (width 0.7) (layer "F.Cu") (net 3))
 (segment (start 145.526 112.19) (end 150.366 112.19) (width 0.7) (layer "F.Cu") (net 3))
 (segment (start 139.216 105.88) (end 145.526 112.19) (width 0.2) (layer "B.Cu") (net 3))
 (segment (start 139.216 98.5) (end 139.216 105.88) (width 0.2) (layer "B.Cu") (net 3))
 (segment (start 96.716 105.92) (end 105.526 114.73) (width 0.2) (layer "B.Cu") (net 17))
 (segment (start 105.526 114.73) (end 137.906 114.73) (width 0.2) (layer "B.Cu") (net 17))
 (segment (start 193.531 100.1) (end 193.531 104.631) (width 0.7) (layer "F.Cu") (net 22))
 (segment (start 193.531 104.631) (end 195.072 106.172) (width 0.7) (layer "F.Cu") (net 22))
 (segment (start 198.611 100.1) (end 198.611 105.173) (width 0.7) (layer "F.Cu") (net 21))
 (segment (start 198.611 105.173) (end 197.612 106.172) (width 0.7) (layer "F.Cu") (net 21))
 (segment (start 207.247 107.72) (end 201.7 107.72) (width 0.7) (layer "F.Cu") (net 18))
 (segment (start 201.7 107.72) (end 200.152 106.172) (width 0.7) (layer "F.Cu") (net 18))
 (segment (start 203.684 110.26) (end 200.152 113.792) (width 0.7) (layer "F.Cu") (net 19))
 (segment (start 207.247 110.26) (end 203.684 110.26) (width 0.7) (layer "F.Cu") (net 19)))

